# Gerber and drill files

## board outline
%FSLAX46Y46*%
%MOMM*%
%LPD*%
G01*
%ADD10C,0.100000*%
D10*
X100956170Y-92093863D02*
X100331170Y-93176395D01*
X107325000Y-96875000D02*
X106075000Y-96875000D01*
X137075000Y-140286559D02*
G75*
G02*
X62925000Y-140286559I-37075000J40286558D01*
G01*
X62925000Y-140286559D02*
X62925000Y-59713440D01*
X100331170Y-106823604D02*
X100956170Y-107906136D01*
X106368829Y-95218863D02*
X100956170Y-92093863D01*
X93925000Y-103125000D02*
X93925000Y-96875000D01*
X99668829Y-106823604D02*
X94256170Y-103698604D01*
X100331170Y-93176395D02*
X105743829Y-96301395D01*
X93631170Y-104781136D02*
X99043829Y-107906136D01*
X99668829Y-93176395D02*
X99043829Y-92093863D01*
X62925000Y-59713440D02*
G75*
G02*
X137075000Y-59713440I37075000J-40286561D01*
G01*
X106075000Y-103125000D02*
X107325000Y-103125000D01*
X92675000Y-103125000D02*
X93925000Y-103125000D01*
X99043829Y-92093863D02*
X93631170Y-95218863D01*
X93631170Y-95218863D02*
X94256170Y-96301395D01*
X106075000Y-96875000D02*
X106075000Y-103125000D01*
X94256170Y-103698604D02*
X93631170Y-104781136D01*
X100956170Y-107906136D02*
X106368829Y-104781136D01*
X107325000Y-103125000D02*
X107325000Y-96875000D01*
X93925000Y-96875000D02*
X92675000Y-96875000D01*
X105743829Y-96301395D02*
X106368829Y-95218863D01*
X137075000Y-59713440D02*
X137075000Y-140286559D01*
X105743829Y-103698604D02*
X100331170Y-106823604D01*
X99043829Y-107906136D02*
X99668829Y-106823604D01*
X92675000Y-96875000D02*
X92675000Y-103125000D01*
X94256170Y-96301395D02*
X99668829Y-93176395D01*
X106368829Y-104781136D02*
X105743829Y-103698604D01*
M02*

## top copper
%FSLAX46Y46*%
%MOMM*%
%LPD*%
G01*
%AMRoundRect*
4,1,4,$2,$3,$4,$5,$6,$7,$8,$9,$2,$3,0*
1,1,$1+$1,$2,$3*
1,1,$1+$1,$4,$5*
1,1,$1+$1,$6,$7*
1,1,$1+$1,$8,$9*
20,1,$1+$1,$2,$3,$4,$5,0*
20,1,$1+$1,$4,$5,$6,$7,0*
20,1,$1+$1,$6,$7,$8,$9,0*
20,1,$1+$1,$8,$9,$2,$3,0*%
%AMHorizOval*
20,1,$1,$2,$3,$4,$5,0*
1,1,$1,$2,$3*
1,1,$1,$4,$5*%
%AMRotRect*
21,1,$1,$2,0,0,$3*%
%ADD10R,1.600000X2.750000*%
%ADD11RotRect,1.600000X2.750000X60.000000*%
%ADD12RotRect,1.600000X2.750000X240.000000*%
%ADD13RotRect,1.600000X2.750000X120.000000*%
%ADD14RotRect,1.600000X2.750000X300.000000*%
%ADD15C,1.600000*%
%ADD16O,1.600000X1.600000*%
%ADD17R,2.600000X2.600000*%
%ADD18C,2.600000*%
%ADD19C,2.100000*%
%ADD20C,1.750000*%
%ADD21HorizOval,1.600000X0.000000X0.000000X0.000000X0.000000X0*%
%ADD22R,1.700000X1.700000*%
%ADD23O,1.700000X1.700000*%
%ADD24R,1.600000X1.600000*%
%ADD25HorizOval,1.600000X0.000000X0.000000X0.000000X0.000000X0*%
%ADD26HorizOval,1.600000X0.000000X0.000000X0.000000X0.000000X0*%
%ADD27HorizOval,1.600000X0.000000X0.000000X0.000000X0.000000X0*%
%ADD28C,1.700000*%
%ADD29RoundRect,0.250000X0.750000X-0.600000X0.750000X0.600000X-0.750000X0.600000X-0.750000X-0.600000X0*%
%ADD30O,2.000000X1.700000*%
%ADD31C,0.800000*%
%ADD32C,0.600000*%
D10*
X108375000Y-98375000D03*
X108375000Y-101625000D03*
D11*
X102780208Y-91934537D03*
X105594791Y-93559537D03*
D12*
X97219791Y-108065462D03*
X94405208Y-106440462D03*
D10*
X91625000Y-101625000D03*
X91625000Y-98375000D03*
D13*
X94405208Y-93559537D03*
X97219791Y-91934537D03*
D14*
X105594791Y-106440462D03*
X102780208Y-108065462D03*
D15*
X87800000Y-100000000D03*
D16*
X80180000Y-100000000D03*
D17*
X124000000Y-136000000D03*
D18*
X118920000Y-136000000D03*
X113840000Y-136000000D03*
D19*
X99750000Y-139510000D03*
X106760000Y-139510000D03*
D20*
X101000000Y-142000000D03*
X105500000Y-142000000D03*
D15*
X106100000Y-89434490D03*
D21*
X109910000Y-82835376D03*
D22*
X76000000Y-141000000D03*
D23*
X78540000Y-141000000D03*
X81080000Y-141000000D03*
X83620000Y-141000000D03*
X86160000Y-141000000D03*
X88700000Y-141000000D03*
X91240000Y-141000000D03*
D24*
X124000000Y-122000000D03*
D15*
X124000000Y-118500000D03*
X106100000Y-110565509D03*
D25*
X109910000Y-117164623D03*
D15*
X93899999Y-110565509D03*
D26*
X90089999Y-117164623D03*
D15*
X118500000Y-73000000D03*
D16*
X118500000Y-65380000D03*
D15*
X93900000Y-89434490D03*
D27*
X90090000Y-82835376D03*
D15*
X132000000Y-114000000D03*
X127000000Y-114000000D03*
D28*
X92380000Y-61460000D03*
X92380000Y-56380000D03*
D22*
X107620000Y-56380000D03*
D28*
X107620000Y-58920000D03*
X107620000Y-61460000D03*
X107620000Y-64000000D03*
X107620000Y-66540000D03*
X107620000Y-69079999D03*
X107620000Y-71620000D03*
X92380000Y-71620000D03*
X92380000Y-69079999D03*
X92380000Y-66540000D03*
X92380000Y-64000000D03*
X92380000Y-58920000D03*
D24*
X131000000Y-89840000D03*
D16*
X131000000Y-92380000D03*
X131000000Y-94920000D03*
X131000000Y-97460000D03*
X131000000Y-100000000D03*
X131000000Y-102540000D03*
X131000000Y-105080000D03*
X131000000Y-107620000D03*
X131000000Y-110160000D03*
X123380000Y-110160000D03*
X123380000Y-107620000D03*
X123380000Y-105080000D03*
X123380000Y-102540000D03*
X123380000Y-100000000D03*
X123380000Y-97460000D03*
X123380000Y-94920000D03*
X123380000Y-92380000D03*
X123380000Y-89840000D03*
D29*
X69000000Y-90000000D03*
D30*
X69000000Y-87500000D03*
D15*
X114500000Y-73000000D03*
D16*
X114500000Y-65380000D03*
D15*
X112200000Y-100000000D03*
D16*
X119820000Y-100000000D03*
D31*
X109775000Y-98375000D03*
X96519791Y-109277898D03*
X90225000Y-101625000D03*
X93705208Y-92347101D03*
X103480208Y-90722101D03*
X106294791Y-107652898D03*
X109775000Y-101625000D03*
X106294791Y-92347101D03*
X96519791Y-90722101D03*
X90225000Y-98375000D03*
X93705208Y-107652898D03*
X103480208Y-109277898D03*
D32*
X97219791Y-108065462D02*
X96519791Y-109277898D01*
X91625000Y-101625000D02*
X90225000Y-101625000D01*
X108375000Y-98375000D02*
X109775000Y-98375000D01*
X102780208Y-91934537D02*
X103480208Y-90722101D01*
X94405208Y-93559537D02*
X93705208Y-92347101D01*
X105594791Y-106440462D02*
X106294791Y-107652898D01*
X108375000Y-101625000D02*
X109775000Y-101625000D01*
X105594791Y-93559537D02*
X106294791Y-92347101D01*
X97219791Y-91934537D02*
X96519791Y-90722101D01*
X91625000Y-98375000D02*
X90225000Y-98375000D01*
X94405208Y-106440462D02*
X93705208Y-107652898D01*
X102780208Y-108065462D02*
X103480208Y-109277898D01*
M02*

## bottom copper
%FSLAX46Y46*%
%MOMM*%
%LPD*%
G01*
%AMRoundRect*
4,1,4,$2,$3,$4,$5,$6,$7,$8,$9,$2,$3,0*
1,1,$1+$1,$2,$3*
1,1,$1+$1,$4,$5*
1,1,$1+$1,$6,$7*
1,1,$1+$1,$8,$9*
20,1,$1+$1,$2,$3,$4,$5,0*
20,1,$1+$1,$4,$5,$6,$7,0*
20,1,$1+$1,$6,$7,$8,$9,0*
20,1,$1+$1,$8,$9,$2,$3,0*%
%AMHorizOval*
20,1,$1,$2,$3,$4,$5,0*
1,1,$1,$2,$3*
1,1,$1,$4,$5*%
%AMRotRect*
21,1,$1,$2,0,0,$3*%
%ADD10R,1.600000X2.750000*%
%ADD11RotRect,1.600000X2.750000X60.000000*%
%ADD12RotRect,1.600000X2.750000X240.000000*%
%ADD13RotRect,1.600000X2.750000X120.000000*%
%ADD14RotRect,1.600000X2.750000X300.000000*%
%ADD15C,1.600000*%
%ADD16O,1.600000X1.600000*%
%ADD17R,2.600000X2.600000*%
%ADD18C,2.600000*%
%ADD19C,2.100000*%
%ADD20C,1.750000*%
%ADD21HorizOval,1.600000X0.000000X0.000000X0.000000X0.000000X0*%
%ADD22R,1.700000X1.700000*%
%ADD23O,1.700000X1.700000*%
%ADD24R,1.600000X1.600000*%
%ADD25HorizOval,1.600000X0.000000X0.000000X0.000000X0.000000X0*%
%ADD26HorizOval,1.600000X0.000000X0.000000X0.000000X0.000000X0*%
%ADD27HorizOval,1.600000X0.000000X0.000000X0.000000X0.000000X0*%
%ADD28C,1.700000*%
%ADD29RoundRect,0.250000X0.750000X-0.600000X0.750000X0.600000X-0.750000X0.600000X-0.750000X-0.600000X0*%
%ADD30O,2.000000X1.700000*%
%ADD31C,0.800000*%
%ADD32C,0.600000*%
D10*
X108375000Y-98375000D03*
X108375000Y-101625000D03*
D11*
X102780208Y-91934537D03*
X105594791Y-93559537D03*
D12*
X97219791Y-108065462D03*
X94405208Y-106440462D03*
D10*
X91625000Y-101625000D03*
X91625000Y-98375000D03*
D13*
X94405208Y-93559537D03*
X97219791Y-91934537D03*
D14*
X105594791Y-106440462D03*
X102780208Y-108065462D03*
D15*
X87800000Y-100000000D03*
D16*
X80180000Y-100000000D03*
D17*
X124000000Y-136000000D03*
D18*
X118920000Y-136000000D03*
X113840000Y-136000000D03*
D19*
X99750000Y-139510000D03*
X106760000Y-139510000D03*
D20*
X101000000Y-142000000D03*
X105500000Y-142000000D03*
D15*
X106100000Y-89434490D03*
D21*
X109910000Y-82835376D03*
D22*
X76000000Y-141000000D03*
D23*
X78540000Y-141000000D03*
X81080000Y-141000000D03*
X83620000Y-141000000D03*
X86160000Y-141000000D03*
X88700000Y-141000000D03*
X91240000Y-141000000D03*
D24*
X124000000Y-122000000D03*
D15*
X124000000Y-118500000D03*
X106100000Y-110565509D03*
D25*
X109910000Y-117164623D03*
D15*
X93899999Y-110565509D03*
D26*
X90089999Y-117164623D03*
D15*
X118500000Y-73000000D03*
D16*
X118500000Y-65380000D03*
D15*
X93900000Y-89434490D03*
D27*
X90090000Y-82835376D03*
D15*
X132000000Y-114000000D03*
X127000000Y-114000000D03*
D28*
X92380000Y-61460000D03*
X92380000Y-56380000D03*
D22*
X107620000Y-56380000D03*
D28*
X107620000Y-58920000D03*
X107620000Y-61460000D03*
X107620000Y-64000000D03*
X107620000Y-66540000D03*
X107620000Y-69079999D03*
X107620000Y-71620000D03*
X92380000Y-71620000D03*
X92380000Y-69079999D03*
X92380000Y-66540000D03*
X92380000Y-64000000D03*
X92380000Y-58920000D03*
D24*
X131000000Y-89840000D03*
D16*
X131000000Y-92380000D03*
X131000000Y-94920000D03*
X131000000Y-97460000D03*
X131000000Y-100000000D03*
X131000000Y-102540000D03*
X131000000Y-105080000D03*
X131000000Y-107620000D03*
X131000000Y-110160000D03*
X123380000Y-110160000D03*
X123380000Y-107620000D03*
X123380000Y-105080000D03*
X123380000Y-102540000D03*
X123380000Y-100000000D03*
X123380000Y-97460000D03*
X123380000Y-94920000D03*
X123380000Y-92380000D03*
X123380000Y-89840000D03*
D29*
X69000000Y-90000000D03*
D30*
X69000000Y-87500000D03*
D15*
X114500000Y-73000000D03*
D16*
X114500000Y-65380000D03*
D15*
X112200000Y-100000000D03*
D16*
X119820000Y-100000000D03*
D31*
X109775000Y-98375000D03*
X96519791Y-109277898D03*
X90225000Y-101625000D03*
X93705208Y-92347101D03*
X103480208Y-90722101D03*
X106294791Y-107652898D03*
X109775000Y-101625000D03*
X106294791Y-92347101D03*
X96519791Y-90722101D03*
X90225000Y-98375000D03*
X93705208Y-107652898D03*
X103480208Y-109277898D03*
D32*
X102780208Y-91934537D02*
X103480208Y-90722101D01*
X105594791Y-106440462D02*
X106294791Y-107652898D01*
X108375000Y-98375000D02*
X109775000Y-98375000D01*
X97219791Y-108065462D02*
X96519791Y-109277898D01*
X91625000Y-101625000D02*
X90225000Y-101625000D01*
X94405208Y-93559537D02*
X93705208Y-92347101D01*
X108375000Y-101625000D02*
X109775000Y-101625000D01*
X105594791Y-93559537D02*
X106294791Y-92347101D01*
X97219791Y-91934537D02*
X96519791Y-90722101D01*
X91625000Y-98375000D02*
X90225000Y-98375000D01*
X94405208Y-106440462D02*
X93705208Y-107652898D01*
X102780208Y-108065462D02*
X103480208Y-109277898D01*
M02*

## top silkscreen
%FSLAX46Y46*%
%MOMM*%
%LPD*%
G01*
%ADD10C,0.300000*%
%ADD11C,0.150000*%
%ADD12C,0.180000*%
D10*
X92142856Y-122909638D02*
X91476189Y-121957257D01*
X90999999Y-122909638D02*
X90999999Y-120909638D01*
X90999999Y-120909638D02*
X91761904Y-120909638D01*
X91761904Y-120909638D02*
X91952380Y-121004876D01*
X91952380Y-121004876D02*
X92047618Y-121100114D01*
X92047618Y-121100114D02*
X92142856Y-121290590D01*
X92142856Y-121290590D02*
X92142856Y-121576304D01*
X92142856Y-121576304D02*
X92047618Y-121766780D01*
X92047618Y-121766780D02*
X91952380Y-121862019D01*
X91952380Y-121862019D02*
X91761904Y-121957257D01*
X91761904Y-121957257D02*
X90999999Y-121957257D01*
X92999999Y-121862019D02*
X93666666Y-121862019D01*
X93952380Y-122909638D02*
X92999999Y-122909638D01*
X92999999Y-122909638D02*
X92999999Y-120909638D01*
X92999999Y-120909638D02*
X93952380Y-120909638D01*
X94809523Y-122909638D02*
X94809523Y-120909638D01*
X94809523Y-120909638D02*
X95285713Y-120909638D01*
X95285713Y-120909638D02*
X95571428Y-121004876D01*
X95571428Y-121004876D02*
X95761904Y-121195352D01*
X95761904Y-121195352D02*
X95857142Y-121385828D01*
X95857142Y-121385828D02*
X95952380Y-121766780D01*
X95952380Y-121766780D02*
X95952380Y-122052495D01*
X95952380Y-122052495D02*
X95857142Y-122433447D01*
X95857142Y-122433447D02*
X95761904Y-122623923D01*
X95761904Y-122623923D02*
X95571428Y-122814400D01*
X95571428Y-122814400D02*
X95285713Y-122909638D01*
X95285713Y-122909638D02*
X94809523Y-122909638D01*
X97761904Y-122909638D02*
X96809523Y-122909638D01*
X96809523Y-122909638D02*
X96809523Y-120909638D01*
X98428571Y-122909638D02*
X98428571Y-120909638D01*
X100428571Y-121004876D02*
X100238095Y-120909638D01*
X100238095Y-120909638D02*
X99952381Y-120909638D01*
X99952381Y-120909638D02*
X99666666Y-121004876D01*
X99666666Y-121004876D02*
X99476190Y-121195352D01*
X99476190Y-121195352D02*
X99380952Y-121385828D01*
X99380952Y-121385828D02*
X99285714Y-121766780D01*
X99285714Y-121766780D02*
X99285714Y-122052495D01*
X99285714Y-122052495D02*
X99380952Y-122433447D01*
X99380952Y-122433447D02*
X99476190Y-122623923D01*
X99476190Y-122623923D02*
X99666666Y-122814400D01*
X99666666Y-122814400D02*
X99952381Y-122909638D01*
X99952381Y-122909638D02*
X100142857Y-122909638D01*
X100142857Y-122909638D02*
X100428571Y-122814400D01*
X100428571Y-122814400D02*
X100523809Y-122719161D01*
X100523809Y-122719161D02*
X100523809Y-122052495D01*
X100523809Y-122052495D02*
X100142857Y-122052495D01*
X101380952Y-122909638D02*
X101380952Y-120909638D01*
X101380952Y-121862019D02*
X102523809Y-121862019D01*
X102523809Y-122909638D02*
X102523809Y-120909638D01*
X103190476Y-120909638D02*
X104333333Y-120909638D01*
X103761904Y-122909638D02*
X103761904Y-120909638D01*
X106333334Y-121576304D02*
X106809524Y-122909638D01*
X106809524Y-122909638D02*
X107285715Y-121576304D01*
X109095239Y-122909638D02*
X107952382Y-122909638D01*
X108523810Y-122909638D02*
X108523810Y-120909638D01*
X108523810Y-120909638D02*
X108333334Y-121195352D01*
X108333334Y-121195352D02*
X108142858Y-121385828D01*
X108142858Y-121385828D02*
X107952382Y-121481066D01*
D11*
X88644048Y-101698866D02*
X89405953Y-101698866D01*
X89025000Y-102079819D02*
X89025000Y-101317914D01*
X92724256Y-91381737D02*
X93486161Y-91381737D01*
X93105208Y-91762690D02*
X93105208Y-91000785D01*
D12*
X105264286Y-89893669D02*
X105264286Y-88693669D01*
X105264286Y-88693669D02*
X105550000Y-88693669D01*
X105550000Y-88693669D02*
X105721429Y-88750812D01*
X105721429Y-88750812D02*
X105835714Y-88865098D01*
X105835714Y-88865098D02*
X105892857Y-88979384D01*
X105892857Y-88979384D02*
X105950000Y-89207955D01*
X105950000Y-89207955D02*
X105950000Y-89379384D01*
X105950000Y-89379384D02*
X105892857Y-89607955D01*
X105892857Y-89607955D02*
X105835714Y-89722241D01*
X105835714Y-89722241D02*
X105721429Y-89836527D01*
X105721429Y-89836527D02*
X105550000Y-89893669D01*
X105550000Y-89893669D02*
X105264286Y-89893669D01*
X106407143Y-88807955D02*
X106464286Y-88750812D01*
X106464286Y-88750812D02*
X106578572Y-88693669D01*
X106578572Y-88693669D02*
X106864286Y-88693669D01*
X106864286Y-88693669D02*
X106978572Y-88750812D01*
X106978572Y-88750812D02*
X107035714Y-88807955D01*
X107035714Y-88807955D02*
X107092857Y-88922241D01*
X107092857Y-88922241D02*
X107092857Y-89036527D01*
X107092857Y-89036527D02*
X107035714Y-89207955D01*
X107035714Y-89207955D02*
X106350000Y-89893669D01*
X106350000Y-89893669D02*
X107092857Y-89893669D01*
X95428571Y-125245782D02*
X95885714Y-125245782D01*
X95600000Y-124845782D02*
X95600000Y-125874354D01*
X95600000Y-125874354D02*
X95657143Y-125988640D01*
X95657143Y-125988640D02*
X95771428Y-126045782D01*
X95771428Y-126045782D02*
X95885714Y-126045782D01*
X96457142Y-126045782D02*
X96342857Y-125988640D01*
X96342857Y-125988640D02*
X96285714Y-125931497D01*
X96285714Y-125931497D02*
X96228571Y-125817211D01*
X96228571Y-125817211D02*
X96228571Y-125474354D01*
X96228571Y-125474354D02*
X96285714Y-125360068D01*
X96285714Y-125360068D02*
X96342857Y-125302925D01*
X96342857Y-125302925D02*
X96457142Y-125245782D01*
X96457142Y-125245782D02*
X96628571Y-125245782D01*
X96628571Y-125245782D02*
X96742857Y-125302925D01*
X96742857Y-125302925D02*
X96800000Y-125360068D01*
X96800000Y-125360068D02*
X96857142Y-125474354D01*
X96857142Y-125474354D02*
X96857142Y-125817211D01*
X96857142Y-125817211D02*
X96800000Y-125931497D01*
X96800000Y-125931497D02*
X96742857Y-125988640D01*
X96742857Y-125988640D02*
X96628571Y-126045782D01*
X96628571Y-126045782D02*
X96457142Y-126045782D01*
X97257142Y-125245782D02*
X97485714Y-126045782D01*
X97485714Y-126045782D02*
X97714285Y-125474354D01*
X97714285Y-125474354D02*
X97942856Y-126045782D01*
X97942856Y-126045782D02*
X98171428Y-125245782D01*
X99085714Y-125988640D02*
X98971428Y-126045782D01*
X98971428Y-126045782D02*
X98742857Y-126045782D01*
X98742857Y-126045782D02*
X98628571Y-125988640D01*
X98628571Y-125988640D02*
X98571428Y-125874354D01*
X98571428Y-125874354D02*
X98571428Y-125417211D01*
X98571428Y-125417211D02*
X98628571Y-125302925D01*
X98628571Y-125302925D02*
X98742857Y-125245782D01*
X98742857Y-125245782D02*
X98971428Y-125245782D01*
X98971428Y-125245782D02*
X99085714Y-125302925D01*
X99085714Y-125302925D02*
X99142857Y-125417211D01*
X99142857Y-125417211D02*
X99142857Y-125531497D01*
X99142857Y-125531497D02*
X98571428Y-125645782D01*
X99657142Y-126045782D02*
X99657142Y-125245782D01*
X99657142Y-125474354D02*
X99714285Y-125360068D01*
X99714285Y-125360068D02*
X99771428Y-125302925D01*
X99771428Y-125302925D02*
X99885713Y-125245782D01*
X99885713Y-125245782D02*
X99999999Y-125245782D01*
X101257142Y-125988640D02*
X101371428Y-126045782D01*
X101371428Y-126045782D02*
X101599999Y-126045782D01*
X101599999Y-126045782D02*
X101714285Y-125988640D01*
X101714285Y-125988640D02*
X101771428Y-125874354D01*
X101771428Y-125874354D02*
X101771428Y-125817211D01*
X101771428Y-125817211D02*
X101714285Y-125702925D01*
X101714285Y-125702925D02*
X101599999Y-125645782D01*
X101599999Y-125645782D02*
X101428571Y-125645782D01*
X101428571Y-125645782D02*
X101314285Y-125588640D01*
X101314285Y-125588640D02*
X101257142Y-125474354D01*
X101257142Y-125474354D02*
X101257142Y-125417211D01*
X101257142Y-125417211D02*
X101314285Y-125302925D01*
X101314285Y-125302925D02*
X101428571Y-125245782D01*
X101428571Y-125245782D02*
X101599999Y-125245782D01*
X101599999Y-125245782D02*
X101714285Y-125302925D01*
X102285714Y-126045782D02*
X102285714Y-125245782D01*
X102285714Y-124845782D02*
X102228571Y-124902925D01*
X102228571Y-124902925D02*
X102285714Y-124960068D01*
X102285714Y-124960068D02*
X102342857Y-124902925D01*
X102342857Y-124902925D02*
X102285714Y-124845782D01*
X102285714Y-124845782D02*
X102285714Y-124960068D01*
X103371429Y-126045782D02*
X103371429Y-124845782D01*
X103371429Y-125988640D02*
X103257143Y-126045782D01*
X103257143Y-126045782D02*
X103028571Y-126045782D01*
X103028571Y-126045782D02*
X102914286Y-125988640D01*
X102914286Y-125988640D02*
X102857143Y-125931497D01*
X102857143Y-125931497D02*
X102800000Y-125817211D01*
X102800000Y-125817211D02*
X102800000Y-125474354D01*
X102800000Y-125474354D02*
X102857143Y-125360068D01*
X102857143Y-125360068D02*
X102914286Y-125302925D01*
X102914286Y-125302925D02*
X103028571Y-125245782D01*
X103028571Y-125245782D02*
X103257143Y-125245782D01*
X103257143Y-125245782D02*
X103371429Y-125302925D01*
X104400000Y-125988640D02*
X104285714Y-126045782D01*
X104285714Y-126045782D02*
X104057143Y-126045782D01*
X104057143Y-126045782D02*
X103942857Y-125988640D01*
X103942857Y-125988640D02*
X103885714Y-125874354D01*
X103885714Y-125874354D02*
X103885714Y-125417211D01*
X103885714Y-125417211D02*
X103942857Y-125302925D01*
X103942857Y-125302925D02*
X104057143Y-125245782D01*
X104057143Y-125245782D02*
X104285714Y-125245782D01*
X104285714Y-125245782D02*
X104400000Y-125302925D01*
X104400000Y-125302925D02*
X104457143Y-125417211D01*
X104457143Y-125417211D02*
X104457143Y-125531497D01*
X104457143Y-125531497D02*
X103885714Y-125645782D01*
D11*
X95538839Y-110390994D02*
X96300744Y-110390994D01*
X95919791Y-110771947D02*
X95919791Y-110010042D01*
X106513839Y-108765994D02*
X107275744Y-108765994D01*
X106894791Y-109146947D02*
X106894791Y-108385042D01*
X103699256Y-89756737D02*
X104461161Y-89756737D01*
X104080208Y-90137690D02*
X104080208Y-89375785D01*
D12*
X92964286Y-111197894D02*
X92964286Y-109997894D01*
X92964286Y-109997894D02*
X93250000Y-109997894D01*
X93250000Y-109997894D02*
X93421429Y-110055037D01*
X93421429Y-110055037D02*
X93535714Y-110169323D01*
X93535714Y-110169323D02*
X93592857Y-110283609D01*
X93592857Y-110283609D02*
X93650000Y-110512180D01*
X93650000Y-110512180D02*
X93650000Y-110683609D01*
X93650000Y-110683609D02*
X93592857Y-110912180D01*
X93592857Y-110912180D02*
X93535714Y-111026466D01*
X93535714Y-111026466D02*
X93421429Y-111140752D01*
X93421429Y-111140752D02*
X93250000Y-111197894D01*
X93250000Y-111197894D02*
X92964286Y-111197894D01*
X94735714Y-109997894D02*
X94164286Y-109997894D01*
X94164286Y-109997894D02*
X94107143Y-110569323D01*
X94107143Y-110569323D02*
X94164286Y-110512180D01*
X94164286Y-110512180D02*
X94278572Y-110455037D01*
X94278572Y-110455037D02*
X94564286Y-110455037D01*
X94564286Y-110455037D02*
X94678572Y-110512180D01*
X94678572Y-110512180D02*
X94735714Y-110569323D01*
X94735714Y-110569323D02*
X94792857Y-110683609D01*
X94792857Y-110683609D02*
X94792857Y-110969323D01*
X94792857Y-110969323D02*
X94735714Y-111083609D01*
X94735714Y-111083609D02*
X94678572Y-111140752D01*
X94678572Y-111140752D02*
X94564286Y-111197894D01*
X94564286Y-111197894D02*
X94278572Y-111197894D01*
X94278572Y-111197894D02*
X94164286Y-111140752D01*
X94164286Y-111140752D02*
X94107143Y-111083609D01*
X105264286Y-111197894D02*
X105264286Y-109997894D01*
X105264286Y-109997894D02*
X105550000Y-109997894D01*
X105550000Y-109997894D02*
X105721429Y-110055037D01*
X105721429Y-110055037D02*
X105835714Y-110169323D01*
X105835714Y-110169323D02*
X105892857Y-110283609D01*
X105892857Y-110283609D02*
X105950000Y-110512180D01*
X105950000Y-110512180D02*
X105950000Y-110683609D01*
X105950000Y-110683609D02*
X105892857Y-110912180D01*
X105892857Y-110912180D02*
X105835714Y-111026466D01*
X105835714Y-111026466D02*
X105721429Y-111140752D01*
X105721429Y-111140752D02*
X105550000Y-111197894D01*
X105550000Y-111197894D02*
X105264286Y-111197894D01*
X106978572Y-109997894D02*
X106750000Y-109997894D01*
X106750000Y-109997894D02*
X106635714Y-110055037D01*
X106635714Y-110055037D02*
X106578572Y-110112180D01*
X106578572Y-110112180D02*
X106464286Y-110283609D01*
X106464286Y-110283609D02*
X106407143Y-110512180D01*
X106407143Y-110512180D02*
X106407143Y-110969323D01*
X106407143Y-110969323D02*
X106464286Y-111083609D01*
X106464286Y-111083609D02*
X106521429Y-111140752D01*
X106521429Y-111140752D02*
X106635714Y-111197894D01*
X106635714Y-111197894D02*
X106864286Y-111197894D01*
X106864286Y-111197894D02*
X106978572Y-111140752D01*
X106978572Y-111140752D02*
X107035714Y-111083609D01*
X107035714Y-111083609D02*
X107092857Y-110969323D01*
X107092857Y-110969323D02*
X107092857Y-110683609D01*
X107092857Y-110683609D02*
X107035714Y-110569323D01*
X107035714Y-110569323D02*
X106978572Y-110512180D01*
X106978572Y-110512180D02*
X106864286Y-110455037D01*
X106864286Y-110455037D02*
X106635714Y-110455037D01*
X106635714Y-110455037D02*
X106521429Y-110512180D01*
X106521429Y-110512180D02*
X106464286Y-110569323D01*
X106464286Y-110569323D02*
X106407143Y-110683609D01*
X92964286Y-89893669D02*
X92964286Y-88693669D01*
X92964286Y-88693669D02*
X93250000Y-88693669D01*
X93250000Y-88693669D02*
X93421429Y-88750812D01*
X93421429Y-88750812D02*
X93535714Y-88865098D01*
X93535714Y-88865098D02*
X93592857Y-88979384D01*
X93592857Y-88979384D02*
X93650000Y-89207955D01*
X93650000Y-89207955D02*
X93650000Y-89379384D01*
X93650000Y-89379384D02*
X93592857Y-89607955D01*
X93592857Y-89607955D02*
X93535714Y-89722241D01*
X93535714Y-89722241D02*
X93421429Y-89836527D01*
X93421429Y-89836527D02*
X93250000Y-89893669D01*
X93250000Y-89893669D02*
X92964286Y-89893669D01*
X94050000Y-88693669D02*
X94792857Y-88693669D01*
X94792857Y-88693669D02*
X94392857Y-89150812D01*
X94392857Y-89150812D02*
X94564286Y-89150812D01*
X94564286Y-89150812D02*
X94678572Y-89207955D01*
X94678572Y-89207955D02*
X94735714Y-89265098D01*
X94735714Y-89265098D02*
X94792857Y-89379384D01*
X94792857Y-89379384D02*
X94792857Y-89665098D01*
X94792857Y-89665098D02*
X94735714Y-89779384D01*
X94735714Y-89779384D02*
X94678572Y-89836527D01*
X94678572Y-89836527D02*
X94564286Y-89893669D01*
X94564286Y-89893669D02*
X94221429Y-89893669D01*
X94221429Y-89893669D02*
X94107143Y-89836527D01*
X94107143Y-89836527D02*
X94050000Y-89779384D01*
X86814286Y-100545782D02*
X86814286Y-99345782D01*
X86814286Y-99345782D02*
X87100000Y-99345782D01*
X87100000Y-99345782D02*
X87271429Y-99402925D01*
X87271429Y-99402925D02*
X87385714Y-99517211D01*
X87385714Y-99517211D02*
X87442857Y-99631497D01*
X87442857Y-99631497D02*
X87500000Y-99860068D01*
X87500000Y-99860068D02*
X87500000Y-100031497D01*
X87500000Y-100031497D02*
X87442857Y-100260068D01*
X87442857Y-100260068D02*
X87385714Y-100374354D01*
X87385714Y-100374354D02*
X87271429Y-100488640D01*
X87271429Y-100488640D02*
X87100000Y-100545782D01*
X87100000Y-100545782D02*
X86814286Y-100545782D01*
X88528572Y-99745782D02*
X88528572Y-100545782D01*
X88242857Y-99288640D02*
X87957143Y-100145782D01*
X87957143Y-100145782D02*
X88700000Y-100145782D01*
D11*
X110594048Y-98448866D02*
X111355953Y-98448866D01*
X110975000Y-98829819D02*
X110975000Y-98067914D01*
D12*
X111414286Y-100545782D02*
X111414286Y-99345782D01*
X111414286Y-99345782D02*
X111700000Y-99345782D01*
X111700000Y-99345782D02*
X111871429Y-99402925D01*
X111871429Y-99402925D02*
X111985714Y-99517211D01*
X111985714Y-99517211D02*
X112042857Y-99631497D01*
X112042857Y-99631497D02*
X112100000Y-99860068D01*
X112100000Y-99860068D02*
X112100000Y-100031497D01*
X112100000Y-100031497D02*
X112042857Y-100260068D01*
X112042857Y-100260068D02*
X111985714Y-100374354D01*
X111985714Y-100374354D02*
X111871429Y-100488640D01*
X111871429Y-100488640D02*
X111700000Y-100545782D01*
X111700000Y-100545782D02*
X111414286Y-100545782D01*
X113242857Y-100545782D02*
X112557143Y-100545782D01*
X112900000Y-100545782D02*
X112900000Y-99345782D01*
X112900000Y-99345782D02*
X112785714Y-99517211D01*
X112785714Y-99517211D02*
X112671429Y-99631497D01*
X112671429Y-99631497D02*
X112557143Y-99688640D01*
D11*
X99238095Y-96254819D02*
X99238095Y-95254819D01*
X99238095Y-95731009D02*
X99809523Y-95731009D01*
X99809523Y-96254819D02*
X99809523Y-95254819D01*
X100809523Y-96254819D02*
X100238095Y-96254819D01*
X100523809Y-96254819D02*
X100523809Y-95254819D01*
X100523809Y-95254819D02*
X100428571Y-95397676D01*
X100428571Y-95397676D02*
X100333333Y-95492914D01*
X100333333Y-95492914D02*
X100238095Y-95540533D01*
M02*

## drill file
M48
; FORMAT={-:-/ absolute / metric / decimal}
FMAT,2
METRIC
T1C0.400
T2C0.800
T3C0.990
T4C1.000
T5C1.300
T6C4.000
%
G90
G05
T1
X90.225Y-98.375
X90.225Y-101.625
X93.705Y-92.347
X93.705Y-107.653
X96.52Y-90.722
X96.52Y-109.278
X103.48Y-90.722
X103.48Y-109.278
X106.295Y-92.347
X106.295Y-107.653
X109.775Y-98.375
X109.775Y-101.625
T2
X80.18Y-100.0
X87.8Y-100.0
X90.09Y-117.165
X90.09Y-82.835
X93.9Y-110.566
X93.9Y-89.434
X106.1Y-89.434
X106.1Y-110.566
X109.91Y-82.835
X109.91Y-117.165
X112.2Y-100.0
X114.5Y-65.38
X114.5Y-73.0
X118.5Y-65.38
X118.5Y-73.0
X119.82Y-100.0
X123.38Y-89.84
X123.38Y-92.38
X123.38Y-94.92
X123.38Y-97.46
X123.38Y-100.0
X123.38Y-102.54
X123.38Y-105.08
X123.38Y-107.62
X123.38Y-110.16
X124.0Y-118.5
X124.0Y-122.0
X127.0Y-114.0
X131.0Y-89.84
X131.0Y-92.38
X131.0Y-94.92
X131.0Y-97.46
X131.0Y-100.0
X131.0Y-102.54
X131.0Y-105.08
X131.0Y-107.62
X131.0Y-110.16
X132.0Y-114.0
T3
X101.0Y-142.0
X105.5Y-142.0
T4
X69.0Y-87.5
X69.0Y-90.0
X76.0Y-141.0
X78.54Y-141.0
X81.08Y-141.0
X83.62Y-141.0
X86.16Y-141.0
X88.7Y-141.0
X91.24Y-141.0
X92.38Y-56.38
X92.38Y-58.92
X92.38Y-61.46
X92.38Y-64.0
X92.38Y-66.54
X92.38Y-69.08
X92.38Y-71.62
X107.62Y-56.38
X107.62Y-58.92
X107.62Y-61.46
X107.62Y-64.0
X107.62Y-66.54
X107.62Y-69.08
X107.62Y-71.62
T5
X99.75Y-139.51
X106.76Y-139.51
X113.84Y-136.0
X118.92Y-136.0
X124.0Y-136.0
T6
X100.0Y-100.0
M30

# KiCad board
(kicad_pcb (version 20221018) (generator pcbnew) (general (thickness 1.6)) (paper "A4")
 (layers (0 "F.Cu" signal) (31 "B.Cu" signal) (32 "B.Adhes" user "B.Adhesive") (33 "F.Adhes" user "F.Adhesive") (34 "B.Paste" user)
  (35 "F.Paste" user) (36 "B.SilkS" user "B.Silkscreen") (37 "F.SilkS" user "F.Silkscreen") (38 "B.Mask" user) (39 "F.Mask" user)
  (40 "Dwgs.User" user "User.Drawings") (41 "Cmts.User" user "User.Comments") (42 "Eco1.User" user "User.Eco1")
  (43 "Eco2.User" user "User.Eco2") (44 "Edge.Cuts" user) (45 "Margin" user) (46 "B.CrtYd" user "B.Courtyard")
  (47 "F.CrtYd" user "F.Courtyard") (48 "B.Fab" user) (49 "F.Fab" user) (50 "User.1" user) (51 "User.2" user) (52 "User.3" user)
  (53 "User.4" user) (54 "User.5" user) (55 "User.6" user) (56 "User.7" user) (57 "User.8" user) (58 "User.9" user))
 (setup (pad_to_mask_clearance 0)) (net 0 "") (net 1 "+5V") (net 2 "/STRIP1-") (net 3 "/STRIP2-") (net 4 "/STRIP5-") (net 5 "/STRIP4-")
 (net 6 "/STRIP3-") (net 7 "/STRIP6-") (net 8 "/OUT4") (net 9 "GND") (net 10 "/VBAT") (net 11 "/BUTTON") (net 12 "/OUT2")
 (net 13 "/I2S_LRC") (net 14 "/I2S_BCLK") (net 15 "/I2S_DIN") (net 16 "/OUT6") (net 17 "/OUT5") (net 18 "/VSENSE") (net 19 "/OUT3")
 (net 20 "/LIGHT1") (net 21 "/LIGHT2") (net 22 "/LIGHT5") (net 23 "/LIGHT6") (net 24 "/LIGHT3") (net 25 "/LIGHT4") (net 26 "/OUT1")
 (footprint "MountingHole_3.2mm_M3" (layer "F.Cu") (at 100 100)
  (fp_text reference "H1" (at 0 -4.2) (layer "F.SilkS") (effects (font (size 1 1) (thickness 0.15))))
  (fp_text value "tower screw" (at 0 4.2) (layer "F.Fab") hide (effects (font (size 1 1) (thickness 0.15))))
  (pad "" np_thru_hole circle (at 0 0) (size 4 4) (drill 4) (layers "*.Cu" "*.Mask")))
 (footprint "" (layer "F.Cu") (at 106.7 100)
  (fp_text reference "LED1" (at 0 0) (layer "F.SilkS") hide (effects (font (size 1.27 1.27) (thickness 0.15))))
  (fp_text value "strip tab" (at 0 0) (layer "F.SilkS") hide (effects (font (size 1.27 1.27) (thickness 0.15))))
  (pad "+" smd rect (at 1.675 -1.625) (size 1.6 2.75) (layers "F.Cu" "F.Mask") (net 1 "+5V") (thermal_bridge_angle 45))
  (pad "+" smd rect (at 1.675 -1.625) (size 1.6 2.75) (layers "B.Cu" "B.Mask") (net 1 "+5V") (thermal_bridge_angle 45))
  (pad "-" smd rect (at 1.675 1.625) (size 1.6 2.75) (layers "F.Cu" "F.Mask") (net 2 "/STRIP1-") (thermal_bridge_angle 45))
  (pad "-" smd rect (at 1.675 1.625) (size 1.6 2.75) (layers "B.Cu" "B.Mask") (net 2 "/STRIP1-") (thermal_bridge_angle 45)))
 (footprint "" (layer "F.Cu") (at 103.35 94.197629)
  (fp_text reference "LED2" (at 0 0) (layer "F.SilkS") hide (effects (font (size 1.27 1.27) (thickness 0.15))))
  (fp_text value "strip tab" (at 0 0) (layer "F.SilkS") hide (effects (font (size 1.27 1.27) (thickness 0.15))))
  (pad "+" smd rect (at -0.569792 -2.263092 60) (size 1.6 2.75) (layers "F.Cu" "F.Mask") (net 1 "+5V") (thermal_bridge_angle 45))
  (pad "+" smd rect (at -0.569792 -2.263092 60) (size 1.6 2.75) (layers "B.Cu" "B.Mask") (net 1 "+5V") (thermal_bridge_angle 45))
  (pad "-" smd rect (at 2.244791 -0.638092 60) (size 1.6 2.75) (layers "F.Cu" "F.Mask") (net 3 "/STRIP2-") (thermal_bridge_angle 45))
  (pad "-" smd rect (at 2.244791 -0.638092 60) (size 1.6 2.75) (layers "B.Cu" "B.Mask") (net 3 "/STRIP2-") (thermal_bridge_angle 45)))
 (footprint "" (layer "F.Cu") (at 96.649999 105.80237)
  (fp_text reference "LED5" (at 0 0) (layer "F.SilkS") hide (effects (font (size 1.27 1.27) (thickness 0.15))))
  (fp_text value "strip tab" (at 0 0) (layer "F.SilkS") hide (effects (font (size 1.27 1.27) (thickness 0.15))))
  (pad "+" smd rect (at 0.569792 2.263092 240) (size 1.6 2.75) (layers "F.Cu" "F.Mask") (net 1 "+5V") (thermal_bridge_angle 45))
  (pad "+" smd rect (at 0.569792 2.263092 240) (size 1.6 2.75) (layers "B.Cu" "B.Mask") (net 1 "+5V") (thermal_bridge_angle 45))
  (pad "-" smd rect (at -2.244791 0.638092 240) (size 1.6 2.75) (layers "F.Cu" "F.Mask") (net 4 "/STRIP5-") (thermal_bridge_angle 45))
  (pad "-" smd rect (at -2.244791 0.638092 240) (size 1.6 2.75) (layers "B.Cu" "B.Mask") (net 4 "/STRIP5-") (thermal_bridge_angle 45)))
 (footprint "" (layer "F.Cu") (at 93.3 100)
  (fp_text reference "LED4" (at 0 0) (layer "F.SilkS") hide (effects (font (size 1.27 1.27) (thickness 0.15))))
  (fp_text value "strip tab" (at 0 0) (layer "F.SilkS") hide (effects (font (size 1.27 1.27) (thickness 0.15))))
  (pad "+" smd rect (at -1.675 1.625 180) (size 1.6 2.75) (layers "F.Cu" "F.Mask") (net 1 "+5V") (thermal_bridge_angle 45))
  (pad "+" smd rect (at -1.675 1.625 180) (size 1.6 2.75) (layers "B.Cu" "B.Mask") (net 1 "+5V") (thermal_bridge_angle 45))
  (pad "-" smd rect (at -1.675 -1.625 180) (size 1.6 2.75) (layers "F.Cu" "F.Mask") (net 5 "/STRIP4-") (thermal_bridge_angle 45))
  (pad "-" smd rect (at -1.675 -1.625 180) (size 1.6 2.75) (layers "B.Cu" "B.Mask") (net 5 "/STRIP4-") (thermal_bridge_angle 45)))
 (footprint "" (layer "F.Cu") (at 96.65 94.197629)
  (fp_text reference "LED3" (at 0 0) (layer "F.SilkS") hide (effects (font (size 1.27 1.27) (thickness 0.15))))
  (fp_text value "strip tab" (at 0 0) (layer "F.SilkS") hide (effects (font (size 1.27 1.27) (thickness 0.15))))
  (pad "+" smd rect (at -2.244792 -0.638092 120) (size 1.6 2.75) (layers "F.Cu" "F.Mask") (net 1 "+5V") (thermal_bridge_angle 45))
  (pad "+" smd rect (at -2.244792 -0.638092 120) (size 1.6 2.75) (layers "B.Cu" "B.Mask") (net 1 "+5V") (thermal_bridge_angle 45))
  (pad "-" smd rect (at 0.569791 -2.263092 120) (size 1.6 2.75) (layers "F.Cu" "F.Mask") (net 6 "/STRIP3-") (thermal_bridge_angle 45))
  (pad "-" smd rect (at 0.569791 -2.263092 120) (size 1.6 2.75) (layers "B.Cu" "B.Mask") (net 6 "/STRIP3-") (thermal_bridge_angle 45)))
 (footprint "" (layer "F.Cu") (at 103.35 105.80237)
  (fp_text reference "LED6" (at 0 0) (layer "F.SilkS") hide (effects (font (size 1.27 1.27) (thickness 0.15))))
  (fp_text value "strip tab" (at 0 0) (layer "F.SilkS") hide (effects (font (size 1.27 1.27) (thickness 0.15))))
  (pad "+" smd rect (at 2.244791 0.638092 300) (size 1.6 2.75) (layers "F.Cu" "F.Mask") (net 1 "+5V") (thermal_bridge_angle 45))
  (pad "+" smd rect (at 2.244791 0.638092 300) (size 1.6 2.75) (layers "B.Cu" "B.Mask") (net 1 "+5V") (thermal_bridge_angle 45))
  (pad "-" smd rect (at -0.569792 2.263092 300) (size 1.6 2.75) (layers "F.Cu" "F.Mask") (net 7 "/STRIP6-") (thermal_bridge_angle 45))
  (pad "-" smd rect (at -0.569792 2.263092 300) (size 1.6 2.75) (layers "B.Cu" "B.Mask") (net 7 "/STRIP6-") (thermal_bridge_angle 45)))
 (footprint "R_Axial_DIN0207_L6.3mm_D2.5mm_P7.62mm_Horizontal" (layer "B.Cu") (at 87.8 100 180)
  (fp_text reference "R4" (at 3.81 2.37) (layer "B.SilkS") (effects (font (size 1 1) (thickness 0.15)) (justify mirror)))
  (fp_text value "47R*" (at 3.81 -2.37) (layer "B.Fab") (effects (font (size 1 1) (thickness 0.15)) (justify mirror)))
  (pad "1" thru_hole circle (at 0 0 180) (size 1.6 1.6) (drill 0.8) (layers "*.Cu" "*.Mask") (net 5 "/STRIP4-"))
  (pad "2" thru_hole oval (at 7.62 0 180) (size 1.6 1.6) (drill 0.8) (layers "*.Cu" "*.Mask") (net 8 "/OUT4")))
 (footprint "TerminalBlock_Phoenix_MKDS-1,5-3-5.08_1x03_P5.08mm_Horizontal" (layer "B.Cu") (at 124 136 180)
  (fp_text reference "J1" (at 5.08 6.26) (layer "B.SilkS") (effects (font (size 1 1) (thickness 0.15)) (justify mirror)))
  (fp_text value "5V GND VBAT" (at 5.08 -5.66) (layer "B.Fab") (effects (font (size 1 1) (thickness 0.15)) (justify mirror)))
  (pad "1" thru_hole rect (at 0 0 180) (size 2.6 2.6) (drill 1.3) (layers "*.Cu" "*.Mask") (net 1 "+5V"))
  (pad "2" thru_hole circle (at 5.08 0 180) (size 2.6 2.6) (drill 1.3) (layers "*.Cu" "*.Mask") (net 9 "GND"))
  (pad "3" thru_hole circle (at 10.16 0 180) (size 2.6 2.6) (drill 1.3) (layers "*.Cu" "*.Mask") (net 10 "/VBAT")))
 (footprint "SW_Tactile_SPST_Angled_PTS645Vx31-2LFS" (layer "B.Cu") (at 101 142)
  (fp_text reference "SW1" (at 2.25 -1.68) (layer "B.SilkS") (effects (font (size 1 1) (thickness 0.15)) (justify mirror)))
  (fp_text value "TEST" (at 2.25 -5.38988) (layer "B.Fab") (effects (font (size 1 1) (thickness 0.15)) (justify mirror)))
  (pad "" thru_hole circle (at -1.25 -2.49) (size 2.1 2.1) (drill 1.3) (layers "*.Cu" "*.Mask"))
  (pad "" thru_hole circle (at 5.76 -2.49) (size 2.1 2.1) (drill 1.3) (layers "*.Cu" "*.Mask"))
  (pad "1" thru_hole circle (at 0 0) (size 1.75 1.75) (drill 0.99) (layers "*.Cu" "*.Mask") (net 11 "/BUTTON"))
  (pad "2" thru_hole circle (at 4.5 0) (size 1.75 1.75) (drill 0.99) (layers "*.Cu" "*.Mask") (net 9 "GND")))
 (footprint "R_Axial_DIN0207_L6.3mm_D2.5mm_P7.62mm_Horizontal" (layer "B.Cu") (at 106.1 89.43449 60)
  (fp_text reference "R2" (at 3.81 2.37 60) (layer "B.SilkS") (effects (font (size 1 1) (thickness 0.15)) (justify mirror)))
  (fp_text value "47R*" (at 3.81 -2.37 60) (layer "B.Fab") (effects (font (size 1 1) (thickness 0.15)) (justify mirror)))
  (pad "1" thru_hole circle (at 0 0 60) (size 1.6 1.6) (drill 0.8) (layers "*.Cu" "*.Mask") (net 3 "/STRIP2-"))
  (pad "2" thru_hole oval (at 7.62 0 60) (size 1.6 1.6) (drill 0.8) (layers "*.Cu" "*.Mask") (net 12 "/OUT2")))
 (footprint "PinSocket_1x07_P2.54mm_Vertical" (layer "B.Cu") (at 76 141 -90)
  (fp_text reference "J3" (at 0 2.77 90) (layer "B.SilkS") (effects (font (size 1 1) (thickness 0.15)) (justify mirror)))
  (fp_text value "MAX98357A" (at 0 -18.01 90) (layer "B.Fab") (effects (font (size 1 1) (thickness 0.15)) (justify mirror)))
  (pad "1" thru_hole rect (at 0 0 270) (size 1.7 1.7) (drill 1) (layers "*.Cu" "*.Mask") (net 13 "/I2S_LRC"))
  (pad "2" thru_hole oval (at 0 -2.54 270) (size 1.7 1.7) (drill 1) (layers "*.Cu" "*.Mask") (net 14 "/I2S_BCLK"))
  (pad "3" thru_hole oval (at 0 -5.08 270) (size 1.7 1.7) (drill 1) (layers "*.Cu" "*.Mask") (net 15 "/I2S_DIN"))
  (pad "4" thru_hole oval (at 0 -7.62 270) (size 1.7 1.7) (drill 1) (layers "*.Cu" "*.Mask"))
  (pad "5" thru_hole oval (at 0 -10.16 270) (size 1.7 1.7) (drill 1) (layers "*.Cu" "*.Mask"))
  (pad "6" thru_hole oval (at 0 -12.7 270) (size 1.7 1.7) (drill 1) (layers "*.Cu" "*.Mask") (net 9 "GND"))
  (pad "7" thru_hole oval (at 0 -15.24 270) (size 1.7 1.7) (drill 1) (layers "*.Cu" "*.Mask") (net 1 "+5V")))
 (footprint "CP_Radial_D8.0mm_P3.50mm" (layer "B.Cu") (at 124 122 90)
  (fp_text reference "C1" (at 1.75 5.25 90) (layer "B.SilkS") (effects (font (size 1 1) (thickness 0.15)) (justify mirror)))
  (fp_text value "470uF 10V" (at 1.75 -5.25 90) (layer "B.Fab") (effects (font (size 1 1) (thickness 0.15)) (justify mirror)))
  (pad "1" thru_hole rect (at 0 0 90) (size 1.6 1.6) (drill 0.8) (layers "*.Cu" "*.Mask") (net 1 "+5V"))
  (pad "2" thru_hole circle (at 3.5 0 90) (size 1.6 1.6) (drill 0.8) (layers "*.Cu" "*.Mask") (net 9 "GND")))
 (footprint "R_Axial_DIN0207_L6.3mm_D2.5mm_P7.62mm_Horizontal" (layer "B.Cu") (at 106.1 110.565509 -60)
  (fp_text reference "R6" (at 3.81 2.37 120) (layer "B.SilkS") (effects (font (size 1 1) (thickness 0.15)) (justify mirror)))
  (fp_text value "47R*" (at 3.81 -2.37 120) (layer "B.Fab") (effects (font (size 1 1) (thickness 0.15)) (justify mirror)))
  (pad "1" thru_hole circle (at 0 0 300) (size 1.6 1.6) (drill 0.8) (layers "*.Cu" "*.Mask") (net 7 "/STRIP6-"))
  (pad "2" thru_hole oval (at 7.62 0 300) (size 1.6 1.6) (drill 0.8) (layers "*.Cu" "*.Mask") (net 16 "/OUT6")))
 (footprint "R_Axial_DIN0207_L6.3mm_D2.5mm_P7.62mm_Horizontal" (layer "B.Cu") (at 93.899999 110.565509 -120)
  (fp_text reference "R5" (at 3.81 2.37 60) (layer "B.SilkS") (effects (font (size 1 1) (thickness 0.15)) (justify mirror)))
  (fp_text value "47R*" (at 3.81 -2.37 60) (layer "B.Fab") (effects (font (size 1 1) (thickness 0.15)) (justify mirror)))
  (pad "1" thru_hole circle (at 0 0 240) (size 1.6 1.6) (drill 0.8) (layers "*.Cu" "*.Mask") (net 4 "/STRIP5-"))
  (pad "2" thru_hole oval (at 7.62 0 240) (size 1.6 1.6) (drill 0.8) (layers "*.Cu" "*.Mask") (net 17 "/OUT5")))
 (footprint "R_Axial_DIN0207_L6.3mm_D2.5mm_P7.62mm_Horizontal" (layer "B.Cu") (at 118.5 73 90)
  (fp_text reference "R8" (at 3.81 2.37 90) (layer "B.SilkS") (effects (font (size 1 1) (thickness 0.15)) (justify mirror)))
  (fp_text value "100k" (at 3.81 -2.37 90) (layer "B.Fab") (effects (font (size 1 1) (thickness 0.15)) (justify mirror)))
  (pad "1" thru_hole circle (at 0 0 90) (size 1.6 1.6) (drill 0.8) (layers "*.Cu" "*.Mask") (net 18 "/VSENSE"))
  (pad "2" thru_hole oval (at 7.62 0 90) (size 1.6 1.6) (drill 0.8) (layers "*.Cu" "*.Mask") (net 9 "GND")))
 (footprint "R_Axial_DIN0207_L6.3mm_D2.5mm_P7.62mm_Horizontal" (layer "B.Cu") (at 93.9 89.43449 120)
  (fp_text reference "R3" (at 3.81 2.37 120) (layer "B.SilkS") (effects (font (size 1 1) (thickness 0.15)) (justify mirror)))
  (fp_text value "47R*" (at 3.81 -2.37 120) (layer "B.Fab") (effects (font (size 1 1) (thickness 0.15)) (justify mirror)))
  (pad "1" thru_hole circle (at 0 0 120) (size 1.6 1.6) (drill 0.8) (layers "*.Cu" "*.Mask") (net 6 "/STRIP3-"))
  (pad "2" thru_hole oval (at 7.62 0 120) (size 1.6 1.6) (drill 0.8) (layers "*.Cu" "*.Mask") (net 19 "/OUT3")))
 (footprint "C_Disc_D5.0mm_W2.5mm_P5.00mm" (layer "B.Cu") (at 132 114 180)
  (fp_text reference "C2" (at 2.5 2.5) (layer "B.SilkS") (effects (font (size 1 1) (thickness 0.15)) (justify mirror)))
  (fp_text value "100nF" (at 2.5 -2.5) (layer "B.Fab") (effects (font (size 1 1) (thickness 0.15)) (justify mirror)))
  (pad "1" thru_hole circle (at 0 0 180) (size 1.6 1.6) (drill 0.8) (layers "*.Cu" "*.Mask") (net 1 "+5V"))
  (pad "2" thru_hole circle (at 5 0 180) (size 1.6 1.6) (drill 0.8) (layers "*.Cu" "*.Mask") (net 9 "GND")))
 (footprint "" (layer "B.Cu") (at 100 64 180)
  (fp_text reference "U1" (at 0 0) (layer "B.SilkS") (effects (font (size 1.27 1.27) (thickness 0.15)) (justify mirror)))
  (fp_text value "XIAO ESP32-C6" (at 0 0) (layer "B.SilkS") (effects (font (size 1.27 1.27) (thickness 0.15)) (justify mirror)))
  (pad "3V3" thru_hole circle (at 7.62 2.54 180) (size 1.7 1.7) (drill 1) (layers "*.Cu" "*.Mask"))
  (pad "5V" thru_hole circle (at 7.62 7.62 180) (size 1.7 1.7) (drill 1) (layers "*.Cu" "*.Mask") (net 1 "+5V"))
  (pad "D0" thru_hole rect (at -7.62 7.62 180) (size 1.7 1.7) (drill 1) (layers "*.Cu" "*.Mask") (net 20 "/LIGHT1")
   (thermal_bridge_angle 45))
  (pad "D1" thru_hole circle (at -7.62 5.08 180) (size 1.7 1.7) (drill 1) (layers "*.Cu" "*.Mask") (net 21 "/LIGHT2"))
  (pad "D2" thru_hole circle (at -7.62 2.54 180) (size 1.7 1.7) (drill 1) (layers "*.Cu" "*.Mask") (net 18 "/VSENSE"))
  (pad "D3" thru_hole circle (at -7.62 0 180) (size 1.7 1.7) (drill 1) (layers "*.Cu" "*.Mask") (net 15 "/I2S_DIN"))
  (pad "D4" thru_hole circle (at -7.62 -2.54 180) (size 1.7 1.7) (drill 1) (layers "*.Cu" "*.Mask") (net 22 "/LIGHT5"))
  (pad "D5" thru_hole circle (at -7.62 -5.079999 180) (size 1.7 1.7) (drill 1) (layers "*.Cu" "*.Mask") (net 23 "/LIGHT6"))
  (pad "D6" thru_hole circle (at -7.62 -7.62 180) (size 1.7 1.7) (drill 1) (layers "*.Cu" "*.Mask") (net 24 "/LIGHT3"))
  (pad "D7" thru_hole circle (at 7.62 -7.62 180) (size 1.7 1.7) (drill 1) (layers "*.Cu" "*.Mask") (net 11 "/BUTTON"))
  (pad "D8" thru_hole circle (at 7.62 -5.079999 180) (size 1.7 1.7) (drill 1) (layers "*.Cu" "*.Mask") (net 14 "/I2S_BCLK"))
  (pad "D9" thru_hole circle (at 7.62 -2.54 180) (size 1.7 1.7) (drill 1) (layers "*.Cu" "*.Mask") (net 13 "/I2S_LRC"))
  (pad "D10" thru_hole circle (at 7.62 0 180) (size 1.7 1.7) (drill 1) (layers "*.Cu" "*.Mask") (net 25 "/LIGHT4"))
  (pad "GND" thru_hole circle (at 7.62 5.08 180) (size 1.7 1.7) (drill 1) (layers "*.Cu" "*.Mask") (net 9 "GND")))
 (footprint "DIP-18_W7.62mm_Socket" (layer "B.Cu") (at 131 89.84 180)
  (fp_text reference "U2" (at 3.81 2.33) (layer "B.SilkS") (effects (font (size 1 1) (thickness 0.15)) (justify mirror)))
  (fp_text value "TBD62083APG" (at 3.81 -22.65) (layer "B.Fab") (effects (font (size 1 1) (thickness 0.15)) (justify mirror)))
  (pad "1" thru_hole rect (at 0 0 180) (size 1.6 1.6) (drill 0.8) (layers "*.Cu" "*.Mask") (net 20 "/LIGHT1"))
  (pad "2" thru_hole oval (at 0 -2.54 180) (size 1.6 1.6) (drill 0.8) (layers "*.Cu" "*.Mask") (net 21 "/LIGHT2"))
  (pad "3" thru_hole oval (at 0 -5.08 180) (size 1.6 1.6) (drill 0.8) (layers "*.Cu" "*.Mask") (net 24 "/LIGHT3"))
  (pad "4" thru_hole oval (at 0 -7.62 180) (size 1.6 1.6) (drill 0.8) (layers "*.Cu" "*.Mask") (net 25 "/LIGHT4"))
  (pad "5" thru_hole oval (at 0 -10.16 180) (size 1.6 1.6) (drill 0.8) (layers "*.Cu" "*.Mask") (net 22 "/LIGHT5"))
  (pad "6" thru_hole oval (at 0 -12.7 180) (size 1.6 1.6) (drill 0.8) (layers "*.Cu" "*.Mask") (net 23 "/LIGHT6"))
  (pad "7" thru_hole oval (at 0 -15.24 180) (size 1.6 1.6) (drill 0.8) (layers "*.Cu" "*.Mask") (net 9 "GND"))
  (pad "8" thru_hole oval (at 0 -17.78 180) (size 1.6 1.6) (drill 0.8) (layers "*.Cu" "*.Mask") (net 9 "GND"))
  (pad "9" thru_hole oval (at 0 -20.32 180) (size 1.6 1.6) (drill 0.8) (layers "*.Cu" "*.Mask") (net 9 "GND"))
  (pad "10" thru_hole oval (at 7.62 -20.32 180) (size 1.6 1.6) (drill 0.8) (layers "*.Cu" "*.Mask") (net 1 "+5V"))
  (pad "11" thru_hole oval (at 7.62 -17.78 180) (size 1.6 1.6) (drill 0.8) (layers "*.Cu" "*.Mask"))
  (pad "12" thru_hole oval (at 7.62 -15.24 180) (size 1.6 1.6) (drill 0.8) (layers "*.Cu" "*.Mask"))
  (pad "13" thru_hole oval (at 7.62 -12.7 180) (size 1.6 1.6) (drill 0.8) (layers "*.Cu" "*.Mask") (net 16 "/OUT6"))
  (pad "14" thru_hole oval (at 7.62 -10.16 180) (size 1.6 1.6) (drill 0.8) (layers "*.Cu" "*.Mask") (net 17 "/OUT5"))
  (pad "15" thru_hole oval (at 7.62 -7.62 180) (size 1.6 1.6) (drill 0.8) (layers "*.Cu" "*.Mask") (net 8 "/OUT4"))
  (pad "16" thru_hole oval (at 7.62 -5.08 180) (size 1.6 1.6) (drill 0.8) (layers "*.Cu" "*.Mask") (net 19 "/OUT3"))
  (pad "17" thru_hole oval (at 7.62 -2.54 180) (size 1.6 1.6) (drill 0.8) (layers "*.Cu" "*.Mask") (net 12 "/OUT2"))
  (pad "18" thru_hole oval (at 7.62 0 180) (size 1.6 1.6) (drill 0.8) (layers "*.Cu" "*.Mask") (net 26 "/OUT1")))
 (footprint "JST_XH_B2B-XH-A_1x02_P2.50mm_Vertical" (layer "B.Cu") (at 69 90 90)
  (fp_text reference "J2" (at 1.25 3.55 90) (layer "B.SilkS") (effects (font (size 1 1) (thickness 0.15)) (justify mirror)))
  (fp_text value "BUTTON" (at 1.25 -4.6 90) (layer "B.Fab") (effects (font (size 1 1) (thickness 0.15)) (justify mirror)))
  (pad "1" thru_hole roundrect (at 0 0 90) (size 1.7 2) (drill 1) (layers "*.Cu" "*.Mask") (roundrect_rratio 0.147059) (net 11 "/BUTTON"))
  (pad "2" thru_hole oval (at 2.5 0 90) (size 1.7 2) (drill 1) (layers "*.Cu" "*.Mask") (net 9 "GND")))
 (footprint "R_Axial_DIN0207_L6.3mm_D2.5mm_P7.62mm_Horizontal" (layer "B.Cu") (at 114.5 73 90)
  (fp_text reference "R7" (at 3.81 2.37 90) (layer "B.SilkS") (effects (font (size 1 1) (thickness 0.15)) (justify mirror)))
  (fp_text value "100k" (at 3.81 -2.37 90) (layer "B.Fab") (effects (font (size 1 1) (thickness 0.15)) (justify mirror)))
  (pad "1" thru_hole circle (at 0 0 90) (size 1.6 1.6) (drill 0.8) (layers "*.Cu" "*.Mask") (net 10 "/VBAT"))
  (pad "2" thru_hole oval (at 7.62 0 90) (size 1.6 1.6) (drill 0.8) (layers "*.Cu" "*.Mask") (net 18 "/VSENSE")))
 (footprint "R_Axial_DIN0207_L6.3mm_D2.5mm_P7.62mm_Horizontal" (layer "B.Cu") (at 112.2 100)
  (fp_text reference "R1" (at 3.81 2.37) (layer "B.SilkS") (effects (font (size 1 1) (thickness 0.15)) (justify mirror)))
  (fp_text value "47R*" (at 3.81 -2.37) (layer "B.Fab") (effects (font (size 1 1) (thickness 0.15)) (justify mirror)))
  (pad "1" thru_hole circle (at 0 0) (size 1.6 1.6) (drill 0.8) (layers "*.Cu" "*.Mask") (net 2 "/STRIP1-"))
  (pad "2" thru_hole oval (at 7.62 0) (size 1.6 1.6) (drill 0.8) (layers "*.Cu" "*.Mask") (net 26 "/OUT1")))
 (gr_line (start 100.95617 92.093863) (end 100.33117 93.176395) (stroke (width 0.1) (type default)) (layer "Edge.Cuts"))
 (gr_line (start 107.325 96.875) (end 106.075 96.875) (stroke (width 0.1) (type default)) (layer "Edge.Cuts"))
 (gr_arc (start 137.075 140.286559) (mid 100 154.75) (end 62.925 140.286559) (stroke (width 0.1) (type default)) (layer "Edge.Cuts"))
 (gr_line (start 62.925 140.286559) (end 62.925 59.71344) (stroke (width 0.1) (type default)) (layer "Edge.Cuts"))
 (gr_line (start 100.33117 106.823604) (end 100.95617 107.906136) (stroke (width 0.1) (type default)) (layer "Edge.Cuts"))
 (gr_line (start 106.368829 95.218863) (end 100.95617 92.093863) (stroke (width 0.1) (type default)) (layer "Edge.Cuts"))
 (gr_line (start 93.925 103.125) (end 93.925 96.875) (stroke (width 0.1) (type default)) (layer "Edge.Cuts"))
 (gr_line (start 99.668829 106.823604) (end 94.25617 103.698604) (stroke (width 0.1) (type default)) (layer "Edge.Cuts"))
 (gr_line (start 100.33117 93.176395) (end 105.743829 96.301395) (stroke (width 0.1) (type default)) (layer "Edge.Cuts"))
 (gr_line (start 93.63117 104.781136) (end 99.043829 107.906136) (stroke (width 0.1) (type default)) (layer "Edge.Cuts"))
 (gr_line (start 99.668829 93.176395) (end 99.043829 92.093863) (stroke (width 0.1) (type default)) (layer "Edge.Cuts"))
 (gr_arc (start 62.925 59.71344) (mid 100 45.25) (end 137.075 59.71344) (stroke (width 0.1) (type default)) (layer "Edge.Cuts"))
 (gr_line (start 106.075 103.125) (end 107.325 103.125) (stroke (width 0.1) (type default)) (layer "Edge.Cuts"))
 (gr_line (start 92.675 103.125) (end 93.925 103.125) (stroke (width 0.1) (type default)) (layer "Edge.Cuts"))
 (gr_line (start 99.043829 92.093863) (end 93.63117 95.218863) (stroke (width 0.1) (type default)) (layer "Edge.Cuts"))
 (gr_line (start 93.63117 95.218863) (end 94.25617 96.301395) (stroke (width 0.1) (type default)) (layer "Edge.Cuts"))
 (gr_line (start 106.075 96.875) (end 106.075 103.125) (stroke (width 0.1) (type default)) (layer "Edge.Cuts"))
 (gr_line (start 94.25617 103.698604) (end 93.63117 104.781136) (stroke (width 0.1) (type default)) (layer "Edge.Cuts"))
 (gr_line (start 100.95617 107.906136) (end 106.368829 104.781136) (stroke (width 0.1) (type default)) (layer "Edge.Cuts"))
 (gr_line (start 107.325 103.125) (end 107.325 96.875) (stroke (width 0.1) (type default)) (layer "Edge.Cuts"))
 (gr_line (start 93.925 96.875) (end 92.675 96.875) (stroke (width 0.1) (type default)) (layer "Edge.Cuts"))
 (gr_line (start 105.743829 96.301395) (end 106.368829 95.218863) (stroke (width 0.1) (type default)) (layer "Edge.Cuts"))
 (gr_line (start 137.075 59.71344) (end 137.075 140.286559) (stroke (width 0.1) (type default)) (layer "Edge.Cuts"))
 (gr_line (start 105.743829 103.698604) (end 100.33117 106.823604) (stroke (width 0.1) (type default)) (layer "Edge.Cuts"))
 (gr_line (start 99.043829 107.906136) (end 99.668829 106.823604) (stroke (width 0.1) (type default)) (layer "Edge.Cuts"))
 (gr_line (start 92.675 96.875) (end 92.675 103.125) (stroke (width 0.1) (type default)) (layer "Edge.Cuts"))
 (gr_line (start 94.25617 96.301395) (end 99.668829 93.176395) (stroke (width 0.1) (type default)) (layer "Edge.Cuts"))
 (gr_line (start 106.368829 104.781136) (end 105.743829 103.698604) (stroke (width 0.1) (type default)) (layer "Edge.Cuts"))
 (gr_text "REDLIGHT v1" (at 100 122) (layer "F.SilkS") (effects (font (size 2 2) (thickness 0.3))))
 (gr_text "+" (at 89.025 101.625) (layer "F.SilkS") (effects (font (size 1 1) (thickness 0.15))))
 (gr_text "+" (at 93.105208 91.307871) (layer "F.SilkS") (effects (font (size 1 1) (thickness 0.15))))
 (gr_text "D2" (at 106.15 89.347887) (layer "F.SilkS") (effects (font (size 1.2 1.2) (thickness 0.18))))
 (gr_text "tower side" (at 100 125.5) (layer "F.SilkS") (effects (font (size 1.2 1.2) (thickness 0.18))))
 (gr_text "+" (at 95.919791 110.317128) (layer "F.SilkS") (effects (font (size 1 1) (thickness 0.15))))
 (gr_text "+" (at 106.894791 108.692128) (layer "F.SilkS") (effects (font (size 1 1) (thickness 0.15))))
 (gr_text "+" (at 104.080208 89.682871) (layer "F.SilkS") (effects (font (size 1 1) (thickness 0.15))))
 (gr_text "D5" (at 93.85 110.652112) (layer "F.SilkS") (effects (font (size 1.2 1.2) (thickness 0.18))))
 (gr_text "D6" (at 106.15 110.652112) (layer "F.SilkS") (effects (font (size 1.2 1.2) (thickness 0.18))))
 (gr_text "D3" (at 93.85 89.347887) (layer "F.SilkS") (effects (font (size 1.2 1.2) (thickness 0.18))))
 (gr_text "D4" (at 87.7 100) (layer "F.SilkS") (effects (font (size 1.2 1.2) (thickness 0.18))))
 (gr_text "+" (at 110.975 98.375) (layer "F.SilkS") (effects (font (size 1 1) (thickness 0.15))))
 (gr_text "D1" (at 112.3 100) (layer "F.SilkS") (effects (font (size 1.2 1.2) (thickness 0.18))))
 (segment (start 97.219791 108.065462) (end 96.519791 109.277898) (width 0.6) (layer "F.Cu") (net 1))
 (segment (start 91.625 101.625) (end 90.225 101.625) (width 0.6) (layer "F.Cu") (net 1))
 (segment (start 108.375 98.375) (end 109.775 98.375) (width 0.6) (layer "F.Cu") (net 1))
 (segment (start 102.780208 91.934537) (end 103.480208 90.722101) (width 0.6) (layer "F.Cu") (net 1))
 (segment (start 94.405208 93.559537) (end 93.705208 92.347101) (width 0.6) (layer "F.Cu") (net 1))
 (segment (start 105.594791 106.440462) (end 106.294791 107.652898) (width 0.6) (layer "F.Cu") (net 1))
 (via (at 109.775 98.375) (size 0.8) (drill 0.4) (layers "F.Cu" "B.Cu") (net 1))
 (via (at 96.519791 109.277898) (size 0.8) (drill 0.4) (layers "F.Cu" "B.Cu") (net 1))
 (via (at 90.225 101.625) (size 0.8) (drill 0.4) (layers "F.Cu" "B.Cu") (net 1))
 (via (at 93.705208 92.347101) (size 0.8) (drill 0.4) (layers "F.Cu" "B.Cu") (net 1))
 (via (at 103.480208 90.722101) (size 0.8) (drill 0.4) (layers "F.Cu" "B.Cu") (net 1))
 (via (at 106.294791 107.652898) (size 0.8) (drill 0.4) (layers "F.Cu" "B.Cu") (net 1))
 (segment (start 102.780208 91.934537) (end 103.480208 90.722101) (width 0.6) (layer "B.Cu") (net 1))
 (segment (start 105.594791 106.440462) (end 106.294791 107.652898) (width 0.6) (layer "B.Cu") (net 1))
 (segment (start 108.375 98.375) (end 109.775 98.375) (width 0.6) (layer "B.Cu") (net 1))
 (segment (start 97.219791 108.065462) (end 96.519791 109.277898) (width 0.6) (layer "B.Cu") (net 1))
 (segment (start 91.625 101.625) (end 90.225 101.625) (width 0.6) (layer "B.Cu") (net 1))
 (segment (start 94.405208 93.559537) (end 93.705208 92.347101) (width 0.6) (layer "B.Cu") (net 1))
 (segment (start 108.375 101.625) (end 109.775 101.625) (width 0.6) (layer "F.Cu") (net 2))
 (via (at 109.775 101.625) (size 0.8) (drill 0.4) (layers "F.Cu" "B.Cu") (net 2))
 (segment (start 108.375 101.625) (end 109.775 101.625) (width 0.6) (layer "B.Cu") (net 2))
 (segment (start 105.594791 93.559537) (end 106.294791 92.347101) (width 0.6) (layer "F.Cu") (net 3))
 (via (at 106.294791 92.347101) (size 0.8) (drill 0.4) (layers "F.Cu" "B.Cu") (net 3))
 (segment (start 105.594791 93.559537) (end 106.294791 92.347101) (width 0.6) (layer "B.Cu") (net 3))
 (segment (start 97.219791 91.934537) (end 96.519791 90.722101) (width 0.6) (layer "F.Cu") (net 6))
 (via (at 96.519791 90.722101) (size 0.8) (drill 0.4) (layers "F.Cu" "B.Cu") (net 6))
 (segment (start 97.219791 91.934537) (end 96.519791 90.722101) (width 0.6) (layer "B.Cu") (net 6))
 (segment (start 91.625 98.375) (end 90.225 98.375) (width 0.6) (layer "F.Cu") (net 5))
 (via (at 90.225 98.375) (size 0.8) (drill 0.4) (layers "F.Cu" "B.Cu") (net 5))
 (segment (start 91.625 98.375) (end 90.225 98.375) (width 0.6) (layer "B.Cu") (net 5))
 (segment (start 94.405208 106.440462) (end 93.705208 107.652898) (width 0.6) (layer "F.Cu") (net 4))
 (via (at 93.705208 107.652898) (size 0.8) (drill 0.4) (layers "F.Cu" "B.Cu") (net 4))
 (segment (start 94.405208 106.440462) (end 93.705208 107.652898) (width 0.6) (layer "B.Cu") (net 4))
 (segment (start 102.780208 108.065462) (end 103.480208 109.277898) (width 0.6) (layer "F.Cu") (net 7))
 (via (at 103.480208 109.277898) (size 0.8) (drill 0.4) (layers "F.Cu" "B.Cu") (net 7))
 (segment (start 102.780208 108.065462) (end 103.480208 109.277898) (width 0.6) (layer "B.Cu") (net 7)))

